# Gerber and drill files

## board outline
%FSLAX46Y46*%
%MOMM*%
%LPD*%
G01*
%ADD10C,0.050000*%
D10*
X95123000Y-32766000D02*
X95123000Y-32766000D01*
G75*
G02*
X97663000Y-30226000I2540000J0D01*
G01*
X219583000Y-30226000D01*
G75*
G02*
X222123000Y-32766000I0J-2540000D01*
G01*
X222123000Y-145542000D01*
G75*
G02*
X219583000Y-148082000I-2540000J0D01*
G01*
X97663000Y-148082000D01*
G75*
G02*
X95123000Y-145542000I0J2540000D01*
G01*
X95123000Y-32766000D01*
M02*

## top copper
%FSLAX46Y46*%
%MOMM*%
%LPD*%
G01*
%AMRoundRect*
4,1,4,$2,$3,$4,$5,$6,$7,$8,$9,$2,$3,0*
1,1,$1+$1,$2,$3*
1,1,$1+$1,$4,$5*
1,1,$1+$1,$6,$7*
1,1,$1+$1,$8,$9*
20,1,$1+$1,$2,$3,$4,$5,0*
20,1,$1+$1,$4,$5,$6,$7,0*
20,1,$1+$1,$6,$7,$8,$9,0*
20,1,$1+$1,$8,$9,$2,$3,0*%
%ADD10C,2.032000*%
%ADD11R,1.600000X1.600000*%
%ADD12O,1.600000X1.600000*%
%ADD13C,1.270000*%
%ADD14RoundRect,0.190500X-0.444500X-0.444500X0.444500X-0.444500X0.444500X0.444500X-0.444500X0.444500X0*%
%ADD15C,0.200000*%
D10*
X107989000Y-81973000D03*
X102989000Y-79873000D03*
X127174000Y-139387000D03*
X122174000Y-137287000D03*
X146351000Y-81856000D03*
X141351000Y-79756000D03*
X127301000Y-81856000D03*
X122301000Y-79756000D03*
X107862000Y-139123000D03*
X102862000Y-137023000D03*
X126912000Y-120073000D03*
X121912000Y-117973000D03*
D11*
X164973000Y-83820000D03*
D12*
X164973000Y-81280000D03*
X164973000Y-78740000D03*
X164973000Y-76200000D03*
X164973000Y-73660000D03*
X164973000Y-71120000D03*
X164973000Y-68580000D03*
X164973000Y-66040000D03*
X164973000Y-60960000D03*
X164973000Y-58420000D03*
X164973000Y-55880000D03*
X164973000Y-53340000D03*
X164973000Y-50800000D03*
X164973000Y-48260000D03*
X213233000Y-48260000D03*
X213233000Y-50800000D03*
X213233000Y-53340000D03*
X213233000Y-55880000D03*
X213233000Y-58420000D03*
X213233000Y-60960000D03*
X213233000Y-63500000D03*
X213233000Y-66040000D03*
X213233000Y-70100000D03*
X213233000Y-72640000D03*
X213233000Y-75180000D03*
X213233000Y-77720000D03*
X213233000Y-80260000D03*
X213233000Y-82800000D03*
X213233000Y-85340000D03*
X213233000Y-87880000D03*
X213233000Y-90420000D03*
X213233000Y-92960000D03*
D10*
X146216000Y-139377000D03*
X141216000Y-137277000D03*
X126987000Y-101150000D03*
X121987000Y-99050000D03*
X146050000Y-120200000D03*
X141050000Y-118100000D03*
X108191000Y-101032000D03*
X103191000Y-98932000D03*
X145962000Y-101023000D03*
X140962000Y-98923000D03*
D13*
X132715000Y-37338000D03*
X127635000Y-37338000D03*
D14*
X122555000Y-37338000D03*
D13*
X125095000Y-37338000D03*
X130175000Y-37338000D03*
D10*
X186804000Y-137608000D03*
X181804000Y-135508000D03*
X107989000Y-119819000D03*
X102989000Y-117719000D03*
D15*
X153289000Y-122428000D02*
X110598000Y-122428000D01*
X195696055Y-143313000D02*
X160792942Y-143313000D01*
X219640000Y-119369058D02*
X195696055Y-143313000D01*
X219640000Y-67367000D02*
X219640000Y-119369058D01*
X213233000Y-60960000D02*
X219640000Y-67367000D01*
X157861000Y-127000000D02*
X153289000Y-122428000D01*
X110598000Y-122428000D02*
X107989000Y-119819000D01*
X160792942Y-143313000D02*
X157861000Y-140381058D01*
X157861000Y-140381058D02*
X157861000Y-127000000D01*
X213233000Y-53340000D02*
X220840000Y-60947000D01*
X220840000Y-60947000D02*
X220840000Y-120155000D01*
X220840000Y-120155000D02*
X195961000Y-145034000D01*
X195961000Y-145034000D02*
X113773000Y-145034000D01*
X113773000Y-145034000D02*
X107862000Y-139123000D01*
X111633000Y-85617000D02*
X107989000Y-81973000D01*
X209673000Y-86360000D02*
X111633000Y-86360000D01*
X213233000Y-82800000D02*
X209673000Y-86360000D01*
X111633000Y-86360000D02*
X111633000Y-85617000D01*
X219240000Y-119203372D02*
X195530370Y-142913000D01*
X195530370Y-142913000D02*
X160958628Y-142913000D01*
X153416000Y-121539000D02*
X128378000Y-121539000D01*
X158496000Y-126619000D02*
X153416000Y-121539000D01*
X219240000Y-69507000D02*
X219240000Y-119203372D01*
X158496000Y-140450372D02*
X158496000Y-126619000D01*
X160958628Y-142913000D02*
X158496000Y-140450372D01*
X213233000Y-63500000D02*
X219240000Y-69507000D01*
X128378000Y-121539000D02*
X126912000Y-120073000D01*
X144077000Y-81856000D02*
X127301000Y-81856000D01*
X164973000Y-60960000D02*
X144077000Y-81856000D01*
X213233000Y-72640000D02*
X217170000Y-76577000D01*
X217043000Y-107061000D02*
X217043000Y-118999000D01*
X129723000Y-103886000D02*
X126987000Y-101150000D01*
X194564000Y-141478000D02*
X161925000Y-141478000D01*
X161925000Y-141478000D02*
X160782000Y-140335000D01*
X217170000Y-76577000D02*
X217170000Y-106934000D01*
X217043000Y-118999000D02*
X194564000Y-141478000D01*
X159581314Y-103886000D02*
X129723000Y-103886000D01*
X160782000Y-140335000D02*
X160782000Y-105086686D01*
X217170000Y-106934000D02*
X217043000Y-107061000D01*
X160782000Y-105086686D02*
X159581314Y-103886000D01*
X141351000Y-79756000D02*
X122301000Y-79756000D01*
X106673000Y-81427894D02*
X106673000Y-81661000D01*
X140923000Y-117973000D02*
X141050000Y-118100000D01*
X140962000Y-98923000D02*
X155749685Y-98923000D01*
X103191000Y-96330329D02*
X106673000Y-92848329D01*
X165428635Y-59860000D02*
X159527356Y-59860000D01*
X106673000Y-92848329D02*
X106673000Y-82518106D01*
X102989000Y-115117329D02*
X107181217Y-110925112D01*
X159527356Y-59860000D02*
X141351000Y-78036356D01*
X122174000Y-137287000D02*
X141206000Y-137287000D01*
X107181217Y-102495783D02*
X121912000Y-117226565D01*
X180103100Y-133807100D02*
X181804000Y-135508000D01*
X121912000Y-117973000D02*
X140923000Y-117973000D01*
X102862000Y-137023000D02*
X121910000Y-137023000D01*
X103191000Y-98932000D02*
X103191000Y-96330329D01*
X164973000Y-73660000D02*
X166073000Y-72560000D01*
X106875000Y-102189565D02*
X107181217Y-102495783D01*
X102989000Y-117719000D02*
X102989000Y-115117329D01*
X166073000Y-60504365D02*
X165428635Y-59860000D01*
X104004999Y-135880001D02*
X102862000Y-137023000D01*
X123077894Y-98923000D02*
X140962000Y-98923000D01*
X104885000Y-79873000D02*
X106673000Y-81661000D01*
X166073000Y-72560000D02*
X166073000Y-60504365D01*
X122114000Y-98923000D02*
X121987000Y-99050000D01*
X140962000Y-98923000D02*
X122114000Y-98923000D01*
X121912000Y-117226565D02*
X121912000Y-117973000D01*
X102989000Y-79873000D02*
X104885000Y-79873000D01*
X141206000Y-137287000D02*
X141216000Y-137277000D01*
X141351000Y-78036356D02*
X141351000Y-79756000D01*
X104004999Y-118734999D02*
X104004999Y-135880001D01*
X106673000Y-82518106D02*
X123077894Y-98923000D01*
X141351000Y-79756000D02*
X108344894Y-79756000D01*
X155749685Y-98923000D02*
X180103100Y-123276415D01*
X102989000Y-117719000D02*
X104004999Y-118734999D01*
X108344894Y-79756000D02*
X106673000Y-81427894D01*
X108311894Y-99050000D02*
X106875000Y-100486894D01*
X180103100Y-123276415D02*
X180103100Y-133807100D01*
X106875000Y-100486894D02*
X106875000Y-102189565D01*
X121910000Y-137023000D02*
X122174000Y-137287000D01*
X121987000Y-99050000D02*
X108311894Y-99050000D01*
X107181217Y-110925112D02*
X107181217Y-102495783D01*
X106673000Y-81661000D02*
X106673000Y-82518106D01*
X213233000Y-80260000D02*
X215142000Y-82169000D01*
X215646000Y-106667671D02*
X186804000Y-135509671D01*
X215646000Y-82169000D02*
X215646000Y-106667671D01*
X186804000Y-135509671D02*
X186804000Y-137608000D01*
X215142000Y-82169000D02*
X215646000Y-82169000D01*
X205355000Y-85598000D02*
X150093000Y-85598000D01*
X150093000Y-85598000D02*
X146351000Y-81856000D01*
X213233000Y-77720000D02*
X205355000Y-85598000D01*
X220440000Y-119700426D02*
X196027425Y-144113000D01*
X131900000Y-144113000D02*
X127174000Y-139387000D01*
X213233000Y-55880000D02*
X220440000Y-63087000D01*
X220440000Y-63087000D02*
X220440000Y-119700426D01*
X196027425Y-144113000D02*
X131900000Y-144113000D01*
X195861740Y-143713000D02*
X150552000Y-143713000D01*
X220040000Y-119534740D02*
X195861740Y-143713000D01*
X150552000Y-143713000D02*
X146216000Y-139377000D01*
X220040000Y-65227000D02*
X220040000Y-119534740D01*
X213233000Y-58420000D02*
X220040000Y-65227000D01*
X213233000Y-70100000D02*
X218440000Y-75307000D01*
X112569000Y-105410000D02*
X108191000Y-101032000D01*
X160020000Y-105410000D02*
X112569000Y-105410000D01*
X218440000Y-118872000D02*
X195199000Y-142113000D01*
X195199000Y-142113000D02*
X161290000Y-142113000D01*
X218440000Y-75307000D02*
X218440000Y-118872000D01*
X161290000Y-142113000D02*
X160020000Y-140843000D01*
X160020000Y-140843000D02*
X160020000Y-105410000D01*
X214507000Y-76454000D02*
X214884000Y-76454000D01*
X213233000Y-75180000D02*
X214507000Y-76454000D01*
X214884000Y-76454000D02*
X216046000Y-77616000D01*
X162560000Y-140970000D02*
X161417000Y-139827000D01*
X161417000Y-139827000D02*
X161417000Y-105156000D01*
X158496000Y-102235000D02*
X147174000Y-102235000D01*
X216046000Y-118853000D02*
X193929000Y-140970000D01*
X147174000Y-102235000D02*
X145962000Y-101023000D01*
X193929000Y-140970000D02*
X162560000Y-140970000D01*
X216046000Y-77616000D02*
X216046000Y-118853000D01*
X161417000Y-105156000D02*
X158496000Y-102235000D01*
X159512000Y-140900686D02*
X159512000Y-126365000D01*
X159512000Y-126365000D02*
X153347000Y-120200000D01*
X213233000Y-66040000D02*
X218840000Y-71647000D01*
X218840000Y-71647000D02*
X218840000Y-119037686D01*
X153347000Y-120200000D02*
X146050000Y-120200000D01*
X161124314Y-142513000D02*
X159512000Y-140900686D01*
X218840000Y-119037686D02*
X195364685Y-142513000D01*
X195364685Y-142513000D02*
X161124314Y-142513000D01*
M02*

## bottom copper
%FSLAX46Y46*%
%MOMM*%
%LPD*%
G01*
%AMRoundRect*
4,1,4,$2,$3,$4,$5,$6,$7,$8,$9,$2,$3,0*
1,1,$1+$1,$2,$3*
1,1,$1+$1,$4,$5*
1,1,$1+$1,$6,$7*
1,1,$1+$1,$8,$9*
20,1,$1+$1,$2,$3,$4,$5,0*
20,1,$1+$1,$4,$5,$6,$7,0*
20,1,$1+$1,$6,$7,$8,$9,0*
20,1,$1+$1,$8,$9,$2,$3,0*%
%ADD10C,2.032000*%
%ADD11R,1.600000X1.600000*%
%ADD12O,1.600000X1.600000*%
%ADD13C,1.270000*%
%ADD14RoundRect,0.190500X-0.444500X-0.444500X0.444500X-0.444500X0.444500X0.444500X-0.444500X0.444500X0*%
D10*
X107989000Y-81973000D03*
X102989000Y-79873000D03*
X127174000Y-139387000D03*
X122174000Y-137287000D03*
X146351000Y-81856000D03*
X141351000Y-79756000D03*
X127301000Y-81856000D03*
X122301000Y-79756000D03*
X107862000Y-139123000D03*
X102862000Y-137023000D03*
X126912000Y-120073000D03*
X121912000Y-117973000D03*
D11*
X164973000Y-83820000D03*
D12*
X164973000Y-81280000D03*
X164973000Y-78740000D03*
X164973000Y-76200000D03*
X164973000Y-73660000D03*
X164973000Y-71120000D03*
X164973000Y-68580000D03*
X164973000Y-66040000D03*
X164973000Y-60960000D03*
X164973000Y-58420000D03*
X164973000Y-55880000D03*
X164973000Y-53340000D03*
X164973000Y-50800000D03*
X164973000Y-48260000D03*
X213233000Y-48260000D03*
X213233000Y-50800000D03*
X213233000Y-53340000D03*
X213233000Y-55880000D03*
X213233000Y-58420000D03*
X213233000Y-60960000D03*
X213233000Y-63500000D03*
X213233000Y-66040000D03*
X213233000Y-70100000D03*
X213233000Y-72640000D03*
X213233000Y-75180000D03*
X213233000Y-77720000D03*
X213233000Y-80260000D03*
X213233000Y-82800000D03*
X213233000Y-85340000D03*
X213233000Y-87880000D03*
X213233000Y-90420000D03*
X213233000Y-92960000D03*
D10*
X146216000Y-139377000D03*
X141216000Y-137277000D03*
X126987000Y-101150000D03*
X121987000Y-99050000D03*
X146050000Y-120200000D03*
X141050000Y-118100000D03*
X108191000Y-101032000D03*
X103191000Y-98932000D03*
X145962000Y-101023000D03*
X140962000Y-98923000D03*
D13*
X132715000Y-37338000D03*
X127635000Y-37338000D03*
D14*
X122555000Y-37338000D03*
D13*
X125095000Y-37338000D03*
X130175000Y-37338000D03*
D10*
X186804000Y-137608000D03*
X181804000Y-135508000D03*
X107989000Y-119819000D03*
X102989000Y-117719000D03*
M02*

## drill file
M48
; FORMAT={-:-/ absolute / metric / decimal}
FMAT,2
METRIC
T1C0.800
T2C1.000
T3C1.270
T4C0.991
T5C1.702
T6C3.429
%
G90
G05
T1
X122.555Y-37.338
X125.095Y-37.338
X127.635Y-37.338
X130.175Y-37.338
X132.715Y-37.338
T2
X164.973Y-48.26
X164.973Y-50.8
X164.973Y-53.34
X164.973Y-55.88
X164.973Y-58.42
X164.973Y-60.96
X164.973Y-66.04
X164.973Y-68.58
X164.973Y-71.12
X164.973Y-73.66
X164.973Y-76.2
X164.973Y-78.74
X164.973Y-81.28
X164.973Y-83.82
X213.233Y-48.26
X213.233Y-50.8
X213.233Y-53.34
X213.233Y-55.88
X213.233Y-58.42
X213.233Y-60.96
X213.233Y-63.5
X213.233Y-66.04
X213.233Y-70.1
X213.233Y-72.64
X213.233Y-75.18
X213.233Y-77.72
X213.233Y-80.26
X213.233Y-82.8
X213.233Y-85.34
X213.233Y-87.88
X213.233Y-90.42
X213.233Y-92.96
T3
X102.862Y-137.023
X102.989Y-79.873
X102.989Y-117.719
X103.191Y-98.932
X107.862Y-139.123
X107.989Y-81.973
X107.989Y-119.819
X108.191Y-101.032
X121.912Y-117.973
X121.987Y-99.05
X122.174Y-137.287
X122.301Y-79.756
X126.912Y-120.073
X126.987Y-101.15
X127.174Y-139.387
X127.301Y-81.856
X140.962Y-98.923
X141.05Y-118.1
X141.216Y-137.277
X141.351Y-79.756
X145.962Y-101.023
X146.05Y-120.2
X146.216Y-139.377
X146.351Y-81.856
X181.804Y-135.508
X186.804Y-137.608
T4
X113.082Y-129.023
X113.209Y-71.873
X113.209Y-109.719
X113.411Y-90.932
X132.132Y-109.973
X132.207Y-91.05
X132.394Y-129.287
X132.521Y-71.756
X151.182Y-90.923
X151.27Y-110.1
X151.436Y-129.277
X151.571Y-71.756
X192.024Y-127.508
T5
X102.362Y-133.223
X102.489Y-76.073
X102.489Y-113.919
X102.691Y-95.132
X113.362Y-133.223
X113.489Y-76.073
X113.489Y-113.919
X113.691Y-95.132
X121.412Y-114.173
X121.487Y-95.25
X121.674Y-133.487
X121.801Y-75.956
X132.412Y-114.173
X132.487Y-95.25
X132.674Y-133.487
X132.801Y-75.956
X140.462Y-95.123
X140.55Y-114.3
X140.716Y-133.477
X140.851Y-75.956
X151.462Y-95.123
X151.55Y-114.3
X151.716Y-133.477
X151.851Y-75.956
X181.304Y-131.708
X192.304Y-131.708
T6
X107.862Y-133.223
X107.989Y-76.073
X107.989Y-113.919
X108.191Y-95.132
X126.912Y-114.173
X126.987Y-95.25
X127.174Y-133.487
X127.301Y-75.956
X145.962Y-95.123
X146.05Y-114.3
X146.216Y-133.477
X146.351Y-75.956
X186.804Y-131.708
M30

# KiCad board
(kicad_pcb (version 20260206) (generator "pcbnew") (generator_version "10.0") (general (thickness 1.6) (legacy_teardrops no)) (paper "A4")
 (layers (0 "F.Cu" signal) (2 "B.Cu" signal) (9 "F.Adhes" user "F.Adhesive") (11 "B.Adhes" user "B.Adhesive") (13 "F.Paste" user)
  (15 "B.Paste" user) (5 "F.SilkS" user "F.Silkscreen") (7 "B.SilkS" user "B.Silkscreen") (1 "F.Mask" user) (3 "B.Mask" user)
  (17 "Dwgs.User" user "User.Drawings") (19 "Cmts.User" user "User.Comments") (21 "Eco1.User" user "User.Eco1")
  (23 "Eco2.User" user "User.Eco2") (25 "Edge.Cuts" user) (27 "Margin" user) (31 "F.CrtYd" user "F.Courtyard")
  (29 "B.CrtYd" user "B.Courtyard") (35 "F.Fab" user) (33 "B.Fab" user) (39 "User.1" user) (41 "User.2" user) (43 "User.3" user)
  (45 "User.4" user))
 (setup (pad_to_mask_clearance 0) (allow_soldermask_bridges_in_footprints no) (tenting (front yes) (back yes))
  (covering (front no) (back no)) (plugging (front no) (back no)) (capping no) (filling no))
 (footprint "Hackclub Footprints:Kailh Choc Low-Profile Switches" (layer "F.Cu") (at 107.989 76.073)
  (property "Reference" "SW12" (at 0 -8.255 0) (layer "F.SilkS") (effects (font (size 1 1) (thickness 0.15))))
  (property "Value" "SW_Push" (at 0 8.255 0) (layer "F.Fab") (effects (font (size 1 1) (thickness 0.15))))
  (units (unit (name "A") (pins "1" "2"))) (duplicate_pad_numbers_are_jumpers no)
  (pad "" np_thru_hole circle (at -5.5 0) (size 1.7018 1.7018) (drill 1.7018) (layers "*.Cu" "*.Mask"))
  (pad "" np_thru_hole circle (at 0 0) (size 3.429 3.429) (drill 3.429) (layers "*.Cu" "*.Mask"))
  (pad "" np_thru_hole circle (at 5.22 -4.2) (size 0.9906 0.9906) (drill 0.9906) (layers "*.Cu" "*.Mask"))
  (pad "" np_thru_hole circle (at 5.5 0) (size 1.7018 1.7018) (drill 1.7018) (layers "*.Cu" "*.Mask"))
  (pad "1" thru_hole circle (at 0 5.9) (size 2.032 2.032) (drill 1.27) (layers "*.Cu" "*.Mask") (remove_unused_layers no) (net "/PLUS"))
  (pad "2" thru_hole circle (at -5 3.8) (size 2.032 2.032) (drill 1.27) (layers "*.Cu" "*.Mask") (remove_unused_layers no) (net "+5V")))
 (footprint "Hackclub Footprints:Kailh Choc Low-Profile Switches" (layer "F.Cu") (at 127.174 133.487)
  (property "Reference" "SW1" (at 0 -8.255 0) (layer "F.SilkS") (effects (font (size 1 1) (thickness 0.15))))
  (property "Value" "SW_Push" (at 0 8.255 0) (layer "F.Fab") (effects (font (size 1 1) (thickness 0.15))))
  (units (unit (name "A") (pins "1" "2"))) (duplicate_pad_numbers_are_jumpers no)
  (pad "" np_thru_hole circle (at -5.5 0) (size 1.7018 1.7018) (drill 1.7018) (layers "*.Cu" "*.Mask"))
  (pad "" np_thru_hole circle (at 0 0) (size 3.429 3.429) (drill 3.429) (layers "*.Cu" "*.Mask"))
  (pad "" np_thru_hole circle (at 5.22 -4.2) (size 0.9906 0.9906) (drill 0.9906) (layers "*.Cu" "*.Mask"))
  (pad "" np_thru_hole circle (at 5.5 0) (size 1.7018 1.7018) (drill 1.7018) (layers "*.Cu" "*.Mask"))
  (pad "1" thru_hole circle (at 0 5.9) (size 2.032 2.032) (drill 1.27) (layers "*.Cu" "*.Mask") (remove_unused_layers no) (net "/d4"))
  (pad "2" thru_hole circle (at -5 3.8) (size 2.032 2.032) (drill 1.27) (layers "*.Cu" "*.Mask") (remove_unused_layers no) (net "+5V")))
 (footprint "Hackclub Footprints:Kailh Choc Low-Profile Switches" (layer "F.Cu") (at 146.351 75.956)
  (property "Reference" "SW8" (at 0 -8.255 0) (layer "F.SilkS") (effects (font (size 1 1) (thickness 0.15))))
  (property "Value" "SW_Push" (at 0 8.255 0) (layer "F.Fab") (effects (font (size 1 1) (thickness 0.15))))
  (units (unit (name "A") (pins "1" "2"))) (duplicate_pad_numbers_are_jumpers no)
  (pad "" np_thru_hole circle (at -5.5 0) (size 1.7018 1.7018) (drill 1.7018) (layers "*.Cu" "*.Mask"))
  (pad "" np_thru_hole circle (at 0 0) (size 3.429 3.429) (drill 3.429) (layers "*.Cu" "*.Mask"))
  (pad "" np_thru_hole circle (at 5.22 -4.2) (size 0.9906 0.9906) (drill 0.9906) (layers "*.Cu" "*.Mask"))
  (pad "" np_thru_hole circle (at 5.5 0) (size 1.7018 1.7018) (drill 1.7018) (layers "*.Cu" "*.Mask"))
  (pad "1" thru_hole circle (at 0 5.9) (size 2.032 2.032) (drill 1.27) (layers "*.Cu" "*.Mask") (remove_unused_layers no) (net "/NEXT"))
  (pad "2" thru_hole circle (at -5 3.8) (size 2.032 2.032) (drill 1.27) (layers "*.Cu" "*.Mask") (remove_unused_layers no) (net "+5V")))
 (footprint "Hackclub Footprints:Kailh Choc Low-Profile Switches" (layer "F.Cu") (at 127.301 75.956)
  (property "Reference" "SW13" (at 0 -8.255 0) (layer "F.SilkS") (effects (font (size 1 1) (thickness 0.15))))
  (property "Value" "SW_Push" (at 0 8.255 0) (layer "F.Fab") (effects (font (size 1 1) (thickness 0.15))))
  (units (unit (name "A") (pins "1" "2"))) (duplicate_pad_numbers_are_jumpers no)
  (pad "" np_thru_hole circle (at -5.5 0) (size 1.7018 1.7018) (drill 1.7018) (layers "*.Cu" "*.Mask"))
  (pad "" np_thru_hole circle (at 0 0) (size 3.429 3.429) (drill 3.429) (layers "*.Cu" "*.Mask"))
  (pad "" np_thru_hole circle (at 5.22 -4.2) (size 0.9906 0.9906) (drill 0.9906) (layers "*.Cu" "*.Mask"))
  (pad "" np_thru_hole circle (at 5.5 0) (size 1.7018 1.7018) (drill 1.7018) (layers "*.Cu" "*.Mask"))
  (pad "1" thru_hole circle (at 0 5.9) (size 2.032 2.032) (drill 1.27) (layers "*.Cu" "*.Mask") (remove_unused_layers no) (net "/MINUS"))
  (pad "2" thru_hole circle (at -5 3.8) (size 2.032 2.032) (drill 1.27) (layers "*.Cu" "*.Mask") (remove_unused_layers no) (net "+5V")))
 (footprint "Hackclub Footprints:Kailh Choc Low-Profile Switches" (layer "F.Cu") (at 107.862 133.223)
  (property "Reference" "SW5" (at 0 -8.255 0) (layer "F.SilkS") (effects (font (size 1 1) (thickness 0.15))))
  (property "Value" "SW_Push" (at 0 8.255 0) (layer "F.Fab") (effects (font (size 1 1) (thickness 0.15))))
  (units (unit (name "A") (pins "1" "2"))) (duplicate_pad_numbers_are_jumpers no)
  (pad "" np_thru_hole circle (at -5.5 0) (size 1.7018 1.7018) (drill 1.7018) (layers "*.Cu" "*.Mask"))
  (pad "" np_thru_hole circle (at 0 0) (size 3.429 3.429) (drill 3.429) (layers "*.Cu" "*.Mask"))
  (pad "" np_thru_hole circle (at 5.22 -4.2) (size 0.9906 0.9906) (drill 0.9906) (layers "*.Cu" "*.Mask"))
  (pad "" np_thru_hole circle (at 5.5 0) (size 1.7018 1.7018) (drill 1.7018) (layers "*.Cu" "*.Mask"))
  (pad "1" thru_hole circle (at 0 5.9) (size 2.032 2.032) (drill 1.27) (layers "*.Cu" "*.Mask") (remove_unused_layers no) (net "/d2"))
  (pad "2" thru_hole circle (at -5 3.8) (size 2.032 2.032) (drill 1.27) (layers "*.Cu" "*.Mask") (remove_unused_layers no) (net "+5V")))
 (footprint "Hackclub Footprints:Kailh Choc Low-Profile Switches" (layer "F.Cu") (at 126.912 114.173)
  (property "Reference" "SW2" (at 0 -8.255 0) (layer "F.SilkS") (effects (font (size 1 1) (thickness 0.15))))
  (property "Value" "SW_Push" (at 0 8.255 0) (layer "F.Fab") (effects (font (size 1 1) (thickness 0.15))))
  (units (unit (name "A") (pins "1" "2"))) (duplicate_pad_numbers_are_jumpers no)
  (pad "" np_thru_hole circle (at -5.5 0) (size 1.7018 1.7018) (drill 1.7018) (layers "*.Cu" "*.Mask"))
  (pad "" np_thru_hole circle (at 0 0) (size 3.429 3.429) (drill 3.429) (layers "*.Cu" "*.Mask"))
  (pad "" np_thru_hole circle (at 5.22 -4.2) (size 0.9906 0.9906) (drill 0.9906) (layers "*.Cu" "*.Mask"))
  (pad "" np_thru_hole circle (at 5.5 0) (size 1.7018 1.7018) (drill 1.7018) (layers "*.Cu" "*.Mask"))
  (pad "1" thru_hole circle (at 0 5.9) (size 2.032 2.032) (drill 1.27) (layers "*.Cu" "*.Mask") (remove_unused_layers no) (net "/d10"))
  (pad "2" thru_hole circle (at -5 3.8) (size 2.032 2.032) (drill 1.27) (layers "*.Cu" "*.Mask") (remove_unused_layers no) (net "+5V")))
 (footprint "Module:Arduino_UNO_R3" (layer "F.Cu") (at 164.973 83.82 90)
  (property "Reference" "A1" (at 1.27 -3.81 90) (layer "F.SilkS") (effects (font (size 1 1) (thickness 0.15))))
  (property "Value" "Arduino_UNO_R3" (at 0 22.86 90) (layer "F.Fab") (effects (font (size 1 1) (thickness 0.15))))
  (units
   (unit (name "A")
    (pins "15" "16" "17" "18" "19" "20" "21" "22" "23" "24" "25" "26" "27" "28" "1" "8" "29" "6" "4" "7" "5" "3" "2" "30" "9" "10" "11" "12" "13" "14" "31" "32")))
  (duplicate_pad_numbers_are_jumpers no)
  (pad "1" thru_hole rect (at 0 0 180) (size 1.6 1.6) (drill 1) (layers "*.Cu" "*.Mask") (remove_unused_layers no)
   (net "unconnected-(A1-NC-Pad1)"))
  (pad "2" thru_hole oval (at 2.54 0 180) (size 1.6 1.6) (drill 1) (layers "*.Cu" "*.Mask") (remove_unused_layers no)
   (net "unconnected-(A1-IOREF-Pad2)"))
  (pad "3" thru_hole oval (at 5.08 0 180) (size 1.6 1.6) (drill 1) (layers "*.Cu" "*.Mask") (remove_unused_layers no)
   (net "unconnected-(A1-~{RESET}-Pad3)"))
  (pad "4" thru_hole oval (at 7.62 0 180) (size 1.6 1.6) (drill 1) (layers "*.Cu" "*.Mask") (remove_unused_layers no)
   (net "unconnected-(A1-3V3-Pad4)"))
  (pad "5" thru_hole oval (at 10.16 0 180) (size 1.6 1.6) (drill 1) (layers "*.Cu" "*.Mask") (remove_unused_layers no) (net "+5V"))
  (pad "6" thru_hole oval (at 12.7 0 180) (size 1.6 1.6) (drill 1) (layers "*.Cu" "*.Mask") (remove_unused_layers no)
   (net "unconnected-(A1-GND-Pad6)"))
  (pad "7" thru_hole oval (at 15.24 0 180) (size 1.6 1.6) (drill 1) (layers "*.Cu" "*.Mask") (remove_unused_layers no) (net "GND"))
  (pad "8" thru_hole oval (at 17.78 0 180) (size 1.6 1.6) (drill 1) (layers "*.Cu" "*.Mask") (remove_unused_layers no)
   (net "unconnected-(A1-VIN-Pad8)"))
  (pad "9" thru_hole oval (at 22.86 0 180) (size 1.6 1.6) (drill 1) (layers "*.Cu" "*.Mask") (remove_unused_layers no) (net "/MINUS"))
  (pad "10" thru_hole oval (at 25.4 0 180) (size 1.6 1.6) (drill 1) (layers "*.Cu" "*.Mask") (remove_unused_layers no)
   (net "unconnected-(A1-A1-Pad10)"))
  (pad "11" thru_hole oval (at 27.94 0 180) (size 1.6 1.6) (drill 1) (layers "*.Cu" "*.Mask") (remove_unused_layers no)
   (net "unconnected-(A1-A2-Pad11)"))
  (pad "12" thru_hole oval (at 30.48 0 180) (size 1.6 1.6) (drill 1) (layers "*.Cu" "*.Mask") (remove_unused_layers no)
   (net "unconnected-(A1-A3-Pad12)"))
  (pad "13" thru_hole oval (at 33.02 0 180) (size 1.6 1.6) (drill 1) (layers "*.Cu" "*.Mask") (remove_unused_layers no)
   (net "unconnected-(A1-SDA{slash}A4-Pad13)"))
  (pad "14" thru_hole oval (at 35.56 0 180) (size 1.6 1.6) (drill 1) (layers "*.Cu" "*.Mask") (remove_unused_layers no)
   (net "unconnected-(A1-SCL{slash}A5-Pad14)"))
  (pad "15" thru_hole oval (at 35.56 48.26 180) (size 1.6 1.6) (drill 1) (layers "*.Cu" "*.Mask") (remove_unused_layers no)
   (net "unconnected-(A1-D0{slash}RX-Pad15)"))
  (pad "16" thru_hole oval (at 33.02 48.26 180) (size 1.6 1.6) (drill 1) (layers "*.Cu" "*.Mask") (remove_unused_layers no)
   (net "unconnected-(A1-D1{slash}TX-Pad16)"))
  (pad "17" thru_hole oval (at 30.48 48.26 180) (size 1.6 1.6) (drill 1) (layers "*.Cu" "*.Mask") (remove_unused_layers no) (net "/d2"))
  (pad "18" thru_hole oval (at 27.94 48.26 180) (size 1.6 1.6) (drill 1) (layers "*.Cu" "*.Mask") (remove_unused_layers no) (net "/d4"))
  (pad "19" thru_hole oval (at 25.4 48.26 180) (size 1.6 1.6) (drill 1) (layers "*.Cu" "*.Mask") (remove_unused_layers no) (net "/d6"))
  (pad "20" thru_hole oval (at 22.86 48.26 180) (size 1.6 1.6) (drill 1) (layers "*.Cu" "*.Mask") (remove_unused_layers no) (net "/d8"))
  (pad "21" thru_hole oval (at 20.32 48.26 180) (size 1.6 1.6) (drill 1) (layers "*.Cu" "*.Mask") (remove_unused_layers no) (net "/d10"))
  (pad "22" thru_hole oval (at 17.78 48.26 180) (size 1.6 1.6) (drill 1) (layers "*.Cu" "*.Mask") (remove_unused_layers no) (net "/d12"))
  (pad "23" thru_hole oval (at 13.72 48.26 180) (size 1.6 1.6) (drill 1) (layers "*.Cu" "*.Mask") (remove_unused_layers no) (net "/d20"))
  (pad "24" thru_hole oval (at 11.18 48.26 180) (size 1.6 1.6) (drill 1) (layers "*.Cu" "*.Mask") (remove_unused_layers no) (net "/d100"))
  (pad "25" thru_hole oval (at 8.64 48.26 180) (size 1.6 1.6) (drill 1) (layers "*.Cu" "*.Mask") (remove_unused_layers no) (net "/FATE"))
  (pad "26" thru_hole oval (at 6.1 48.26 180) (size 1.6 1.6) (drill 1) (layers "*.Cu" "*.Mask") (remove_unused_layers no) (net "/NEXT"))
  (pad "27" thru_hole oval (at 3.56 48.26 180) (size 1.6 1.6) (drill 1) (layers "*.Cu" "*.Mask") (remove_unused_layers no) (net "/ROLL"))
  (pad "28" thru_hole oval (at 1.02 48.26 180) (size 1.6 1.6) (drill 1) (layers "*.Cu" "*.Mask") (remove_unused_layers no) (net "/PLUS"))
  (pad "29" thru_hole oval (at -1.52 48.26 180) (size 1.6 1.6) (drill 1) (layers "*.Cu" "*.Mask") (remove_unused_layers no)
   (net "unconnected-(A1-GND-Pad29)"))
  (pad "30" thru_hole oval (at -4.06 48.26 180) (size 1.6 1.6) (drill 1) (layers "*.Cu" "*.Mask") (remove_unused_layers no)
   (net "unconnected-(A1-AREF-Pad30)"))
  (pad "31" thru_hole oval (at -6.6 48.26 180) (size 1.6 1.6) (drill 1) (layers "*.Cu" "*.Mask") (remove_unused_layers no)
   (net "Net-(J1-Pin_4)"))
  (pad "32" thru_hole oval (at -9.14 48.26 180) (size 1.6 1.6) (drill 1) (layers "*.Cu" "*.Mask") (remove_unused_layers no)
   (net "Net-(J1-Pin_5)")))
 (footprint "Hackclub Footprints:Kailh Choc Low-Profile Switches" (layer "F.Cu") (at 146.216 133.477)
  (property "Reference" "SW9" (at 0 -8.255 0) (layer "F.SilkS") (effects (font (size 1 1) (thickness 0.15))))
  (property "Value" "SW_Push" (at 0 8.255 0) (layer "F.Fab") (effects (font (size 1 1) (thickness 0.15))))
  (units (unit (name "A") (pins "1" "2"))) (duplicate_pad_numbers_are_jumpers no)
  (pad "" np_thru_hole circle (at -5.5 0) (size 1.7018 1.7018) (drill 1.7018) (layers "*.Cu" "*.Mask"))
  (pad "" np_thru_hole circle (at 0 0) (size 3.429 3.429) (drill 3.429) (layers "*.Cu" "*.Mask"))
  (pad "" np_thru_hole circle (at 5.22 -4.2) (size 0.9906 0.9906) (drill 0.9906) (layers "*.Cu" "*.Mask"))
  (pad "" np_thru_hole circle (at 5.5 0) (size 1.7018 1.7018) (drill 1.7018) (layers "*.Cu" "*.Mask"))
  (pad "1" thru_hole circle (at 0 5.9) (size 2.032 2.032) (drill 1.27) (layers "*.Cu" "*.Mask") (remove_unused_layers no) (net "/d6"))
  (pad "2" thru_hole circle (at -5 3.8) (size 2.032 2.032) (drill 1.27) (layers "*.Cu" "*.Mask") (remove_unused_layers no) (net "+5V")))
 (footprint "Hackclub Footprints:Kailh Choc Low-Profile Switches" (layer "F.Cu") (at 126.987 95.25)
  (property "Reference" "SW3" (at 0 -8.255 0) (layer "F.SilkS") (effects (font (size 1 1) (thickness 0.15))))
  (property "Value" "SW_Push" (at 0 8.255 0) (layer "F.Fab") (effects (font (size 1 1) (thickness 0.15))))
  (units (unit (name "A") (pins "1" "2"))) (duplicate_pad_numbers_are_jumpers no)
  (pad "" np_thru_hole circle (at -5.5 0) (size 1.7018 1.7018) (drill 1.7018) (layers "*.Cu" "*.Mask"))
  (pad "" np_thru_hole circle (at 0 0) (size 3.429 3.429) (drill 3.429) (layers "*.Cu" "*.Mask"))
  (pad "" np_thru_hole circle (at 5.22 -4.2) (size 0.9906 0.9906) (drill 0.9906) (layers "*.Cu" "*.Mask"))
  (pad "" np_thru_hole circle (at 5.5 0) (size 1.7018 1.7018) (drill 1.7018) (layers "*.Cu" "*.Mask"))
  (pad "1" thru_hole circle (at 0 5.9) (size 2.032 2.032) (drill 1.27) (layers "*.Cu" "*.Mask") (remove_unused_layers no) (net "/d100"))
  (pad "2" thru_hole circle (at -5 3.8) (size 2.032 2.032) (drill 1.27) (layers "*.Cu" "*.Mask") (remove_unused_layers no) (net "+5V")))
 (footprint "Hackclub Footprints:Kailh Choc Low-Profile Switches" (layer "F.Cu") (at 146.05 114.3)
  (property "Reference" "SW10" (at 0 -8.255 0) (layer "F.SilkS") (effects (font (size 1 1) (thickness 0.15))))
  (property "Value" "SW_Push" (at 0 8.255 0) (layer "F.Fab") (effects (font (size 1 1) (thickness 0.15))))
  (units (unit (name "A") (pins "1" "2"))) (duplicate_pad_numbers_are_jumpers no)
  (pad "" np_thru_hole circle (at -5.5 0) (size 1.7018 1.7018) (drill 1.7018) (layers "*.Cu" "*.Mask"))
  (pad "" np_thru_hole circle (at 0 0) (size 3.429 3.429) (drill 3.429) (layers "*.Cu" "*.Mask"))
  (pad "" np_thru_hole circle (at 5.22 -4.2) (size 0.9906 0.9906) (drill 0.9906) (layers "*.Cu" "*.Mask"))
  (pad "" np_thru_hole circle (at 5.5 0) (size 1.7018 1.7018) (drill 1.7018) (layers "*.Cu" "*.Mask"))
  (pad "1" thru_hole circle (at 0 5.9) (size 2.032 2.032) (drill 1.27) (layers "*.Cu" "*.Mask") (remove_unused_layers no) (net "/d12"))
  (pad "2" thru_hole circle (at -5 3.8) (size 2.032 2.032) (drill 1.27) (layers "*.Cu" "*.Mask") (remove_unused_layers no) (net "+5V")))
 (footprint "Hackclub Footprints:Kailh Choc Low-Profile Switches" (layer "F.Cu") (at 108.191 95.132)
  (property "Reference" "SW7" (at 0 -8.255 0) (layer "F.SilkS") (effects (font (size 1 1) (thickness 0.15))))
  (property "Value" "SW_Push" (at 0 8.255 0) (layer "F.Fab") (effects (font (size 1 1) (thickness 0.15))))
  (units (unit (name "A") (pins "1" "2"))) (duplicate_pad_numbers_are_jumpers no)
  (pad "" np_thru_hole circle (at -5.5 0) (size 1.7018 1.7018) (drill 1.7018) (layers "*.Cu" "*.Mask"))
  (pad "" np_thru_hole circle (at 0 0) (size 3.429 3.429) (drill 3.429) (layers "*.Cu" "*.Mask"))
  (pad "" np_thru_hole circle (at 5.22 -4.2) (size 0.9906 0.9906) (drill 0.9906) (layers "*.Cu" "*.Mask"))
  (pad "" np_thru_hole circle (at 5.5 0) (size 1.7018 1.7018) (drill 1.7018) (layers "*.Cu" "*.Mask"))
  (pad "1" thru_hole circle (at 0 5.9) (size 2.032 2.032) (drill 1.27) (layers "*.Cu" "*.Mask") (remove_unused_layers no) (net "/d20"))
  (pad "2" thru_hole circle (at -5 3.8) (size 2.032 2.032) (drill 1.27) (layers "*.Cu" "*.Mask") (remove_unused_layers no) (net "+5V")))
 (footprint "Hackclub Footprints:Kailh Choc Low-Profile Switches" (layer "F.Cu") (at 145.962 95.123)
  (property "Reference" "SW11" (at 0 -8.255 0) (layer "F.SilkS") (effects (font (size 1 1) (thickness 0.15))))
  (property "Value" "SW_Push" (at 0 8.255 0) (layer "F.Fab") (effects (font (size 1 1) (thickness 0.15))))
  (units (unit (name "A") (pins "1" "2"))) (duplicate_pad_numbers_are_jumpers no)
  (pad "" np_thru_hole circle (at -5.5 0) (size 1.7018 1.7018) (drill 1.7018) (layers "*.Cu" "*.Mask"))
  (pad "" np_thru_hole circle (at 0 0) (size 3.429 3.429) (drill 3.429) (layers "*.Cu" "*.Mask"))
  (pad "" np_thru_hole circle (at 5.22 -4.2) (size 0.9906 0.9906) (drill 0.9906) (layers "*.Cu" "*.Mask"))
  (pad "" np_thru_hole circle (at 5.5 0) (size 1.7018 1.7018) (drill 1.7018) (layers "*.Cu" "*.Mask"))
  (pad "1" thru_hole circle (at 0 5.9) (size 2.032 2.032) (drill 1.27) (layers "*.Cu" "*.Mask") (remove_unused_layers no) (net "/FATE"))
  (pad "2" thru_hole circle (at -5 3.8) (size 2.032 2.032) (drill 1.27) (layers "*.Cu" "*.Mask") (remove_unused_layers no) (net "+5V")))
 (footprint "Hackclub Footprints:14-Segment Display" (layer "F.Cu") (at 127.635 48.768)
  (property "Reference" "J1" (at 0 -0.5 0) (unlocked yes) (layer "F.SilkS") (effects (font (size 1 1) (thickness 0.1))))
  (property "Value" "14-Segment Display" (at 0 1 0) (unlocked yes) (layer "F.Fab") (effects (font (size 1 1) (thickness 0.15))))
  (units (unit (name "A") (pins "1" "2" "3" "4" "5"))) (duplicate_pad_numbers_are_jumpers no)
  (pad "9" thru_hole circle (at 5.08 -11.43) (size 1.27 1.27) (drill 0.8) (layers "*.Cu" "*.Mask") (remove_unused_layers no)
   (thermal_bridge_angle 90))
  (pad "GND" thru_hole circle (at 0 -11.43) (size 1.27 1.27) (drill 0.8) (layers "*.Cu" "*.Mask") (remove_unused_layers no)
   (thermal_bridge_angle 90))
  (pad "SCL" thru_hole roundrect (at -5.08 -11.43) (size 1.27 1.27) (drill 0.8) (layers "*.Cu" "*.Mask") (remove_unused_layers no)
   (roundrect_rratio 0.15))
  (pad "SDA" thru_hole circle (at -2.54 -11.43) (size 1.27 1.27) (drill 0.8) (layers "*.Cu" "*.Mask") (remove_unused_layers no)
   (thermal_bridge_angle 90))
  (pad "VCC" thru_hole circle (at 2.54 -11.43) (size 1.27 1.27) (drill 0.8) (layers "*.Cu" "*.Mask") (remove_unused_layers no)
   (thermal_bridge_angle 90)))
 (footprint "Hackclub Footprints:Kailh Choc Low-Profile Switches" (layer "F.Cu") (at 186.804 131.708)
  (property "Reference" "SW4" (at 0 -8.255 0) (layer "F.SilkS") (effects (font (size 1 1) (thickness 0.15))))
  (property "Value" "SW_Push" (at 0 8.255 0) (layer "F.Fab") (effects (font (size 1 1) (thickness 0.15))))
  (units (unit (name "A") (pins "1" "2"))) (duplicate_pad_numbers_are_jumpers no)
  (pad "" np_thru_hole circle (at -5.5 0) (size 1.7018 1.7018) (drill 1.7018) (layers "*.Cu" "*.Mask"))
  (pad "" np_thru_hole circle (at 0 0) (size 3.429 3.429) (drill 3.429) (layers "*.Cu" "*.Mask"))
  (pad "" np_thru_hole circle (at 5.22 -4.2) (size 0.9906 0.9906) (drill 0.9906) (layers "*.Cu" "*.Mask"))
  (pad "" np_thru_hole circle (at 5.5 0) (size 1.7018 1.7018) (drill 1.7018) (layers "*.Cu" "*.Mask"))
  (pad "1" thru_hole circle (at 0 5.9) (size 2.032 2.032) (drill 1.27) (layers "*.Cu" "*.Mask") (remove_unused_layers no) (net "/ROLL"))
  (pad "2" thru_hole circle (at -5 3.8) (size 2.032 2.032) (drill 1.27) (layers "*.Cu" "*.Mask") (remove_unused_layers no) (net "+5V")))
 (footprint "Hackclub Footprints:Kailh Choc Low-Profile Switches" (layer "F.Cu") (at 107.989 113.919)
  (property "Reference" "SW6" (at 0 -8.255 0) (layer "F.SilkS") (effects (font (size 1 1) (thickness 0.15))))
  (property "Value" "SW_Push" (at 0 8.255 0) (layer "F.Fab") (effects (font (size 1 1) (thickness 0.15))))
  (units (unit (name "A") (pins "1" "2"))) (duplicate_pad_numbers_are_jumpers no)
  (pad "" np_thru_hole circle (at -5.5 0) (size 1.7018 1.7018) (drill 1.7018) (layers "*.Cu" "*.Mask"))
  (pad "" np_thru_hole circle (at 0 0) (size 3.429 3.429) (drill 3.429) (layers "*.Cu" "*.Mask"))
  (pad "" np_thru_hole circle (at 5.22 -4.2) (size 0.9906 0.9906) (drill 0.9906) (layers "*.Cu" "*.Mask"))
  (pad "" np_thru_hole circle (at 5.5 0) (size 1.7018 1.7018) (drill 1.7018) (layers "*.Cu" "*.Mask"))
  (pad "1" thru_hole circle (at 0 5.9) (size 2.032 2.032) (drill 1.27) (layers "*.Cu" "*.Mask") (remove_unused_layers no) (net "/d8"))
  (pad "2" thru_hole circle (at -5 3.8) (size 2.032 2.032) (drill 1.27) (layers "*.Cu" "*.Mask") (remove_unused_layers no) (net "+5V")))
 (gr_rect (start 95.123 30.226) (end 222.123 148.082) (radius 2.54) (stroke (width 0.05) (type solid)) (fill no) (layer "Edge.Cuts"))
 (segment (start 153.289 122.428) (end 110.598 122.428) (width 0.2) (layer "F.Cu") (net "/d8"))
 (segment (start 195.696055 143.313) (end 160.792942 143.313) (width 0.2) (layer "F.Cu") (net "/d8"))
 (segment (start 219.64 119.369058) (end 195.696055 143.313) (width 0.2) (layer "F.Cu") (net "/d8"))
 (segment (start 219.64 67.367) (end 219.64 119.369058) (width 0.2) (layer "F.Cu") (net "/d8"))
 (segment (start 213.233 60.96) (end 219.64 67.367) (width 0.2) (layer "F.Cu") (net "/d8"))
 (segment (start 157.861 127) (end 153.289 122.428) (width 0.2) (layer "F.Cu") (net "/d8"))
 (segment (start 110.598 122.428) (end 107.989 119.819) (width 0.2) (layer "F.Cu") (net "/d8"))
 (segment (start 160.792942 143.313) (end 157.861 140.381058) (width 0.2) (layer "F.Cu") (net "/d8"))
 (segment (start 157.861 140.381058) (end 157.861 127) (width 0.2) (layer "F.Cu") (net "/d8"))
 (segment (start 213.233 53.34) (end 220.84 60.947) (width 0.2) (layer "F.Cu") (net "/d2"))
 (segment (start 220.84 60.947) (end 220.84 120.155) (width 0.2) (layer "F.Cu") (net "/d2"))
 (segment (start 220.84 120.155) (end 195.961 145.034) (width 0.2) (layer "F.Cu") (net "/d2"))
 (segment (start 195.961 145.034) (end 113.773 145.034) (width 0.2) (layer "F.Cu") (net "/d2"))
 (segment (start 113.773 145.034) (end 107.862 139.123) (width 0.2) (layer "F.Cu") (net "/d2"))
 (segment (start 111.633 85.617) (end 107.989 81.973) (width 0.2) (layer "F.Cu") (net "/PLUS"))
 (segment (start 209.673 86.36) (end 111.633 86.36) (width 0.2) (layer "F.Cu") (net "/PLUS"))
 (segment (start 213.233 82.8) (end 209.673 86.36) (width 0.2) (layer "F.Cu") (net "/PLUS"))
 (segment (start 111.633 86.36) (end 111.633 85.617) (width 0.2) (layer "F.Cu") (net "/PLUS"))
 (segment (start 219.24 119.203372) (end 195.53037 142.913) (width 0.2) (layer "F.Cu") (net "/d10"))
 (segment (start 195.53037 142.913) (end 160.958628 142.913) (width 0.2) (layer "F.Cu") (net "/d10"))
 (segment (start 153.416 121.539) (end 128.378 121.539) (width 0.2) (layer "F.Cu") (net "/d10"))
 (segment (start 158.496 126.619) (end 153.416 121.539) (width 0.2) (layer "F.Cu") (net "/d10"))
 (segment (start 219.24 69.507) (end 219.24 119.203372) (width 0.2) (layer "F.Cu") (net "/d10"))
 (segment (start 158.496 140.450372) (end 158.496 126.619) (width 0.2) (layer "F.Cu") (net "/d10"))
 (segment (start 160.958628 142.913) (end 158.496 140.450372) (width 0.2) (layer "F.Cu") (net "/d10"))
 (segment (start 213.233 63.5) (end 219.24 69.507) (width 0.2) (layer "F.Cu") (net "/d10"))
 (segment (start 128.378 121.539) (end 126.912 120.073) (width 0.2) (layer "F.Cu") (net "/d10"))
 (segment (start 144.077 81.856) (end 127.301 81.856) (width 0.2) (layer "F.Cu") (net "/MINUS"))
 (segment (start 164.973 60.96) (end 144.077 81.856) (width 0.2) (layer "F.Cu") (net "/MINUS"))
 (segment (start 213.233 72.64) (end 217.17 76.577) (width 0.2) (layer "F.Cu") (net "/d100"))
 (segment (start 217.043 107.061) (end 217.043 118.999) (width 0.2) (layer "F.Cu") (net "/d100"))
 (segment (start 129.723 103.886) (end 126.987 101.15) (width 0.2) (layer "F.Cu") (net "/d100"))
 (segment (start 194.564 141.478) (end 161.925 141.478) (width 0.2) (layer "F.Cu") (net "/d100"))
 (segment (start 161.925 141.478) (end 160.782 140.335) (width 0.2) (layer "F.Cu") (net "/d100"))
 (segment (start 217.17 76.577) (end 217.17 106.934) (width 0.2) (layer "F.Cu") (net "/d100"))
 (segment (start 217.043 118.999) (end 194.564 141.478) (width 0.2) (layer "F.Cu") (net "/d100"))
 (segment (start 159.581314 103.886) (end 129.723 103.886) (width 0.2) (layer "F.Cu") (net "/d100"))
 (segment (start 160.782 140.335) (end 160.782 105.086686) (width 0.2) (layer "F.Cu") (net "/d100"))
 (segment (start 217.17 106.934) (end 217.043 107.061) (width 0.2) (layer "F.Cu") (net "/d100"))
 (segment (start 160.782 105.086686) (end 159.581314 103.886) (width 0.2) (layer "F.Cu") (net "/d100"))
 (segment (start 141.351 79.756) (end 122.301 79.756) (width 0.2) (layer "F.Cu") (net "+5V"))
 (segment (start 106.673 81.427894) (end 106.673 81.661) (width 0.2) (layer "F.Cu") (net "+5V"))
 (segment (start 140.923 117.973) (end 141.05 118.1) (width 0.2) (layer "F.Cu") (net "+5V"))
 (segment (start 140.962 98.923) (end 155.749685 98.923) (width 0.2) (layer "F.Cu") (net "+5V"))
 (segment (start 103.191 96.330329) (end 106.673 92.848329) (width 0.2) (layer "F.Cu") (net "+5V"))
 (segment (start 165.428635 59.86) (end 159.527356 59.86) (width 0.2) (layer "F.Cu") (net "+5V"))
 (segment (start 106.673 92.848329) (end 106.673 82.518106) (width 0.2) (layer "F.Cu") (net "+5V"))
 (segment (start 102.989 115.117329) (end 107.181217 110.925112) (width 0.2) (layer "F.Cu") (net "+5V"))
 (segment (start 159.527356 59.86) (end 141.351 78.036356) (width 0.2) (layer "F.Cu") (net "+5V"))
 (segment (start 122.174 137.287) (end 141.206 137.287) (width 0.2) (layer "F.Cu") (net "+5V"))
 (segment (start 107.181217 102.495783) (end 121.912 117.226565) (width 0.2) (layer "F.Cu") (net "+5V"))
 (segment (start 180.1031 133.8071) (end 181.804 135.508) (width 0.2) (layer "F.Cu") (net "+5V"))
 (segment (start 121.912 117.973) (end 140.923 117.973) (width 0.2) (layer "F.Cu") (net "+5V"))
 (segment (start 102.862 137.023) (end 121.91 137.023) (width 0.2) (layer "F.Cu") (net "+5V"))
 (segment (start 103.191 98.932) (end 103.191 96.330329) (width 0.2) (layer "F.Cu") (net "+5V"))
 (segment (start 164.973 73.66) (end 166.073 72.56) (width 0.2) (layer "F.Cu") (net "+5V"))
 (segment (start 106.875 102.189565) (end 107.181217 102.495783) (width 0.2) (layer "F.Cu") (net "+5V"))
 (segment (start 102.989 117.719) (end 102.989 115.117329) (width 0.2) (layer "F.Cu") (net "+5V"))
 (segment (start 166.073 60.504365) (end 165.428635 59.86) (width 0.2) (layer "F.Cu") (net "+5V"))
 (segment (start 104.004999 135.880001) (end 102.862 137.023) (width 0.2) (layer "F.Cu") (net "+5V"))
 (segment (start 123.077894 98.923) (end 140.962 98.923) (width 0.2) (layer "F.Cu") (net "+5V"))
 (segment (start 104.885 79.873) (end 106.673 81.661) (width 0.2) (layer "F.Cu") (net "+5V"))
 (segment (start 166.073 72.56) (end 166.073 60.504365) (width 0.2) (layer "F.Cu") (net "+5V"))
 (segment (start 122.114 98.923) (end 121.987 99.05) (width 0.2) (layer "F.Cu") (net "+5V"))
 (segment (start 140.962 98.923) (end 122.114 98.923) (width 0.2) (layer "F.Cu") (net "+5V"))
 (segment (start 121.912 117.226565) (end 121.912 117.973) (width 0.2) (layer "F.Cu") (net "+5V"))
 (segment (start 102.989 79.873) (end 104.885 79.873) (width 0.2) (layer "F.Cu") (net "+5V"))
 (segment (start 141.206 137.287) (end 141.216 137.277) (width 0.2) (layer "F.Cu") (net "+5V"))
 (segment (start 141.351 78.036356) (end 141.351 79.756) (width 0.2) (layer "F.Cu") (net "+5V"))
 (segment (start 104.004999 118.734999) (end 104.004999 135.880001) (width 0.2) (layer "F.Cu") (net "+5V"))
 (segment (start 106.673 82.518106) (end 123.077894 98.923) (width 0.2) (layer "F.Cu") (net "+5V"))
 (segment (start 141.351 79.756) (end 108.344894 79.756) (width 0.2) (layer "F.Cu") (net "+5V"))
 (segment (start 155.749685 98.923) (end 180.1031 123.276415) (width 0.2) (layer "F.Cu") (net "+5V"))
 (segment (start 102.989 117.719) (end 104.004999 118.734999) (width 0.2) (layer "F.Cu") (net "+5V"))
 (segment (start 108.344894 79.756) (end 106.673 81.427894) (width 0.2) (layer "F.Cu") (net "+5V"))
 (segment (start 108.311894 99.05) (end 106.875 100.486894) (width 0.2) (layer "F.Cu") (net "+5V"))
 (segment (start 180.1031 123.276415) (end 180.1031 133.8071) (width 0.2) (layer "F.Cu") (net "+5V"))
 (segment (start 106.875 100.486894) (end 106.875 102.189565) (width 0.2) (layer "F.Cu") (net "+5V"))
 (segment (start 121.91 137.023) (end 122.174 137.287) (width 0.2) (layer "F.Cu") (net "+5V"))
 (segment (start 121.987 99.05) (end 108.311894 99.05) (width 0.2) (layer "F.Cu") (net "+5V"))
 (segment (start 107.181217 110.925112) (end 107.181217 102.495783) (width 0.2) (layer "F.Cu") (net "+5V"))
 (segment (start 106.673 81.661) (end 106.673 82.518106) (width 0.2) (layer "F.Cu") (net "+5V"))
 (segment (start 213.233 80.26) (end 215.142 82.169) (width 0.2) (layer "F.Cu") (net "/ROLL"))
 (segment (start 215.646 106.667671) (end 186.804 135.509671) (width 0.2) (layer "F.Cu") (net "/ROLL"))
 (segment (start 215.646 82.169) (end 215.646 106.667671) (width 0.2) (layer "F.Cu") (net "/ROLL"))
 (segment (start 186.804 135.509671) (end 186.804 137.608) (width 0.2) (layer "F.Cu") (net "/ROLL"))
 (segment (start 215.142 82.169) (end 215.646 82.169) (width 0.2) (layer "F.Cu") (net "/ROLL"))
 (segment (start 205.355 85.598) (end 150.093 85.598) (width 0.2) (layer "F.Cu") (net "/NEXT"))
 (segment (start 150.093 85.598) (end 146.351 81.856) (width 0.2) (layer "F.Cu") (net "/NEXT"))
 (segment (start 213.233 77.72) (end 205.355 85.598) (width 0.2) (layer "F.Cu") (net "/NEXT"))
 (segment (start 220.44 119.700426) (end 196.027425 144.113) (width 0.2) (layer "F.Cu") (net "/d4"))
 (segment (start 131.9 144.113) (end 127.174 139.387) (width 0.2) (layer "F.Cu") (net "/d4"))
 (segment (start 213.233 55.88) (end 220.44 63.087) (width 0.2) (layer "F.Cu") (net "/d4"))
 (segment (start 220.44 63.087) (end 220.44 119.700426) (width 0.2) (layer "F.Cu") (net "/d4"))
 (segment (start 196.027425 144.113) (end 131.9 144.113) (width 0.2) (layer "F.Cu") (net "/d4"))
 (segment (start 195.86174 143.713) (end 150.552 143.713) (width 0.2) (layer "F.Cu") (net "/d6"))
 (segment (start 220.04 119.53474) (end 195.86174 143.713) (width 0.2) (layer "F.Cu") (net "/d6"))
 (segment (start 150.552 143.713) (end 146.216 139.377) (width 0.2) (layer "F.Cu") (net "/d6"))
 (segment (start 220.04 65.227) (end 220.04 119.53474) (width 0.2) (layer "F.Cu") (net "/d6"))
 (segment (start 213.233 58.42) (end 220.04 65.227) (width 0.2) (layer "F.Cu") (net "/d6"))
 (segment (start 213.233 70.1) (end 218.44 75.307) (width 0.2) (layer "F.Cu") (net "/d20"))
 (segment (start 112.569 105.41) (end 108.191 101.032) (width 0.2) (layer "F.Cu") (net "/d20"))
 (segment (start 160.02 105.41) (end 112.569 105.41) (width 0.2) (layer "F.Cu") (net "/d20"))
 (segment (start 218.44 118.872) (end 195.199 142.113) (width 0.2) (layer "F.Cu") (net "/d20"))
 (segment (start 195.199 142.113) (end 161.29 142.113) (width 0.2) (layer "F.Cu") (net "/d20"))
 (segment (start 218.44 75.307) (end 218.44 118.872) (width 0.2) (layer "F.Cu") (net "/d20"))
 (segment (start 161.29 142.113) (end 160.02 140.843) (width 0.2) (layer "F.Cu") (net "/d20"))
 (segment (start 160.02 140.843) (end 160.02 105.41) (width 0.2) (layer "F.Cu") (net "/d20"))
 (segment (start 214.507 76.454) (end 214.884 76.454) (width 0.2) (layer "F.Cu") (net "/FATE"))
 (segment (start 213.233 75.18) (end 214.507 76.454) (width 0.2) (layer "F.Cu") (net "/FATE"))
 (segment (start 214.884 76.454) (end 216.046 77.616) (width 0.2) (layer "F.Cu") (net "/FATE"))
 (segment (start 162.56 140.97) (end 161.417 139.827) (width 0.2) (layer "F.Cu") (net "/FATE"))
 (segment (start 161.417 139.827) (end 161.417 105.156) (width 0.2) (layer "F.Cu") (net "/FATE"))
 (segment (start 158.496 102.235) (end 147.174 102.235) (width 0.2) (layer "F.Cu") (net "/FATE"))
 (segment (start 216.046 118.853) (end 193.929 140.97) (width 0.2) (layer "F.Cu") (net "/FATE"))
 (segment (start 147.174 102.235) (end 145.962 101.023) (width 0.2) (layer "F.Cu") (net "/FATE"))
 (segment (start 193.929 140.97) (end 162.56 140.97) (width 0.2) (layer "F.Cu") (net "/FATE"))
 (segment (start 216.046 77.616) (end 216.046 118.853) (width 0.2) (layer "F.Cu") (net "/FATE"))
 (segment (start 161.417 105.156) (end 158.496 102.235) (width 0.2) (layer "F.Cu") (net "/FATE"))
 (segment (start 159.512 140.900686) (end 159.512 126.365) (width 0.2) (layer "F.Cu") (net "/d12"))
 (segment (start 159.512 126.365) (end 153.347 120.2) (width 0.2) (layer "F.Cu") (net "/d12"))
 (segment (start 213.233 66.04) (end 218.84 71.647) (width 0.2) (layer "F.Cu") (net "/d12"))
 (segment (start 218.84 71.647) (end 218.84 119.037686) (width 0.2) (layer "F.Cu") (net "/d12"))
 (segment (start 153.347 120.2) (end 146.05 120.2) (width 0.2) (layer "F.Cu") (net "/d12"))
 (segment (start 161.124314 142.513) (end 159.512 140.900686) (width 0.2) (layer "F.Cu") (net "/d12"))
 (segment (start 218.84 119.037686) (end 195.364685 142.513) (width 0.2) (layer "F.Cu") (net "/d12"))
 (segment (start 195.364685 142.513) (end 161.124314 142.513) (width 0.2) (layer "F.Cu") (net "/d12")))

